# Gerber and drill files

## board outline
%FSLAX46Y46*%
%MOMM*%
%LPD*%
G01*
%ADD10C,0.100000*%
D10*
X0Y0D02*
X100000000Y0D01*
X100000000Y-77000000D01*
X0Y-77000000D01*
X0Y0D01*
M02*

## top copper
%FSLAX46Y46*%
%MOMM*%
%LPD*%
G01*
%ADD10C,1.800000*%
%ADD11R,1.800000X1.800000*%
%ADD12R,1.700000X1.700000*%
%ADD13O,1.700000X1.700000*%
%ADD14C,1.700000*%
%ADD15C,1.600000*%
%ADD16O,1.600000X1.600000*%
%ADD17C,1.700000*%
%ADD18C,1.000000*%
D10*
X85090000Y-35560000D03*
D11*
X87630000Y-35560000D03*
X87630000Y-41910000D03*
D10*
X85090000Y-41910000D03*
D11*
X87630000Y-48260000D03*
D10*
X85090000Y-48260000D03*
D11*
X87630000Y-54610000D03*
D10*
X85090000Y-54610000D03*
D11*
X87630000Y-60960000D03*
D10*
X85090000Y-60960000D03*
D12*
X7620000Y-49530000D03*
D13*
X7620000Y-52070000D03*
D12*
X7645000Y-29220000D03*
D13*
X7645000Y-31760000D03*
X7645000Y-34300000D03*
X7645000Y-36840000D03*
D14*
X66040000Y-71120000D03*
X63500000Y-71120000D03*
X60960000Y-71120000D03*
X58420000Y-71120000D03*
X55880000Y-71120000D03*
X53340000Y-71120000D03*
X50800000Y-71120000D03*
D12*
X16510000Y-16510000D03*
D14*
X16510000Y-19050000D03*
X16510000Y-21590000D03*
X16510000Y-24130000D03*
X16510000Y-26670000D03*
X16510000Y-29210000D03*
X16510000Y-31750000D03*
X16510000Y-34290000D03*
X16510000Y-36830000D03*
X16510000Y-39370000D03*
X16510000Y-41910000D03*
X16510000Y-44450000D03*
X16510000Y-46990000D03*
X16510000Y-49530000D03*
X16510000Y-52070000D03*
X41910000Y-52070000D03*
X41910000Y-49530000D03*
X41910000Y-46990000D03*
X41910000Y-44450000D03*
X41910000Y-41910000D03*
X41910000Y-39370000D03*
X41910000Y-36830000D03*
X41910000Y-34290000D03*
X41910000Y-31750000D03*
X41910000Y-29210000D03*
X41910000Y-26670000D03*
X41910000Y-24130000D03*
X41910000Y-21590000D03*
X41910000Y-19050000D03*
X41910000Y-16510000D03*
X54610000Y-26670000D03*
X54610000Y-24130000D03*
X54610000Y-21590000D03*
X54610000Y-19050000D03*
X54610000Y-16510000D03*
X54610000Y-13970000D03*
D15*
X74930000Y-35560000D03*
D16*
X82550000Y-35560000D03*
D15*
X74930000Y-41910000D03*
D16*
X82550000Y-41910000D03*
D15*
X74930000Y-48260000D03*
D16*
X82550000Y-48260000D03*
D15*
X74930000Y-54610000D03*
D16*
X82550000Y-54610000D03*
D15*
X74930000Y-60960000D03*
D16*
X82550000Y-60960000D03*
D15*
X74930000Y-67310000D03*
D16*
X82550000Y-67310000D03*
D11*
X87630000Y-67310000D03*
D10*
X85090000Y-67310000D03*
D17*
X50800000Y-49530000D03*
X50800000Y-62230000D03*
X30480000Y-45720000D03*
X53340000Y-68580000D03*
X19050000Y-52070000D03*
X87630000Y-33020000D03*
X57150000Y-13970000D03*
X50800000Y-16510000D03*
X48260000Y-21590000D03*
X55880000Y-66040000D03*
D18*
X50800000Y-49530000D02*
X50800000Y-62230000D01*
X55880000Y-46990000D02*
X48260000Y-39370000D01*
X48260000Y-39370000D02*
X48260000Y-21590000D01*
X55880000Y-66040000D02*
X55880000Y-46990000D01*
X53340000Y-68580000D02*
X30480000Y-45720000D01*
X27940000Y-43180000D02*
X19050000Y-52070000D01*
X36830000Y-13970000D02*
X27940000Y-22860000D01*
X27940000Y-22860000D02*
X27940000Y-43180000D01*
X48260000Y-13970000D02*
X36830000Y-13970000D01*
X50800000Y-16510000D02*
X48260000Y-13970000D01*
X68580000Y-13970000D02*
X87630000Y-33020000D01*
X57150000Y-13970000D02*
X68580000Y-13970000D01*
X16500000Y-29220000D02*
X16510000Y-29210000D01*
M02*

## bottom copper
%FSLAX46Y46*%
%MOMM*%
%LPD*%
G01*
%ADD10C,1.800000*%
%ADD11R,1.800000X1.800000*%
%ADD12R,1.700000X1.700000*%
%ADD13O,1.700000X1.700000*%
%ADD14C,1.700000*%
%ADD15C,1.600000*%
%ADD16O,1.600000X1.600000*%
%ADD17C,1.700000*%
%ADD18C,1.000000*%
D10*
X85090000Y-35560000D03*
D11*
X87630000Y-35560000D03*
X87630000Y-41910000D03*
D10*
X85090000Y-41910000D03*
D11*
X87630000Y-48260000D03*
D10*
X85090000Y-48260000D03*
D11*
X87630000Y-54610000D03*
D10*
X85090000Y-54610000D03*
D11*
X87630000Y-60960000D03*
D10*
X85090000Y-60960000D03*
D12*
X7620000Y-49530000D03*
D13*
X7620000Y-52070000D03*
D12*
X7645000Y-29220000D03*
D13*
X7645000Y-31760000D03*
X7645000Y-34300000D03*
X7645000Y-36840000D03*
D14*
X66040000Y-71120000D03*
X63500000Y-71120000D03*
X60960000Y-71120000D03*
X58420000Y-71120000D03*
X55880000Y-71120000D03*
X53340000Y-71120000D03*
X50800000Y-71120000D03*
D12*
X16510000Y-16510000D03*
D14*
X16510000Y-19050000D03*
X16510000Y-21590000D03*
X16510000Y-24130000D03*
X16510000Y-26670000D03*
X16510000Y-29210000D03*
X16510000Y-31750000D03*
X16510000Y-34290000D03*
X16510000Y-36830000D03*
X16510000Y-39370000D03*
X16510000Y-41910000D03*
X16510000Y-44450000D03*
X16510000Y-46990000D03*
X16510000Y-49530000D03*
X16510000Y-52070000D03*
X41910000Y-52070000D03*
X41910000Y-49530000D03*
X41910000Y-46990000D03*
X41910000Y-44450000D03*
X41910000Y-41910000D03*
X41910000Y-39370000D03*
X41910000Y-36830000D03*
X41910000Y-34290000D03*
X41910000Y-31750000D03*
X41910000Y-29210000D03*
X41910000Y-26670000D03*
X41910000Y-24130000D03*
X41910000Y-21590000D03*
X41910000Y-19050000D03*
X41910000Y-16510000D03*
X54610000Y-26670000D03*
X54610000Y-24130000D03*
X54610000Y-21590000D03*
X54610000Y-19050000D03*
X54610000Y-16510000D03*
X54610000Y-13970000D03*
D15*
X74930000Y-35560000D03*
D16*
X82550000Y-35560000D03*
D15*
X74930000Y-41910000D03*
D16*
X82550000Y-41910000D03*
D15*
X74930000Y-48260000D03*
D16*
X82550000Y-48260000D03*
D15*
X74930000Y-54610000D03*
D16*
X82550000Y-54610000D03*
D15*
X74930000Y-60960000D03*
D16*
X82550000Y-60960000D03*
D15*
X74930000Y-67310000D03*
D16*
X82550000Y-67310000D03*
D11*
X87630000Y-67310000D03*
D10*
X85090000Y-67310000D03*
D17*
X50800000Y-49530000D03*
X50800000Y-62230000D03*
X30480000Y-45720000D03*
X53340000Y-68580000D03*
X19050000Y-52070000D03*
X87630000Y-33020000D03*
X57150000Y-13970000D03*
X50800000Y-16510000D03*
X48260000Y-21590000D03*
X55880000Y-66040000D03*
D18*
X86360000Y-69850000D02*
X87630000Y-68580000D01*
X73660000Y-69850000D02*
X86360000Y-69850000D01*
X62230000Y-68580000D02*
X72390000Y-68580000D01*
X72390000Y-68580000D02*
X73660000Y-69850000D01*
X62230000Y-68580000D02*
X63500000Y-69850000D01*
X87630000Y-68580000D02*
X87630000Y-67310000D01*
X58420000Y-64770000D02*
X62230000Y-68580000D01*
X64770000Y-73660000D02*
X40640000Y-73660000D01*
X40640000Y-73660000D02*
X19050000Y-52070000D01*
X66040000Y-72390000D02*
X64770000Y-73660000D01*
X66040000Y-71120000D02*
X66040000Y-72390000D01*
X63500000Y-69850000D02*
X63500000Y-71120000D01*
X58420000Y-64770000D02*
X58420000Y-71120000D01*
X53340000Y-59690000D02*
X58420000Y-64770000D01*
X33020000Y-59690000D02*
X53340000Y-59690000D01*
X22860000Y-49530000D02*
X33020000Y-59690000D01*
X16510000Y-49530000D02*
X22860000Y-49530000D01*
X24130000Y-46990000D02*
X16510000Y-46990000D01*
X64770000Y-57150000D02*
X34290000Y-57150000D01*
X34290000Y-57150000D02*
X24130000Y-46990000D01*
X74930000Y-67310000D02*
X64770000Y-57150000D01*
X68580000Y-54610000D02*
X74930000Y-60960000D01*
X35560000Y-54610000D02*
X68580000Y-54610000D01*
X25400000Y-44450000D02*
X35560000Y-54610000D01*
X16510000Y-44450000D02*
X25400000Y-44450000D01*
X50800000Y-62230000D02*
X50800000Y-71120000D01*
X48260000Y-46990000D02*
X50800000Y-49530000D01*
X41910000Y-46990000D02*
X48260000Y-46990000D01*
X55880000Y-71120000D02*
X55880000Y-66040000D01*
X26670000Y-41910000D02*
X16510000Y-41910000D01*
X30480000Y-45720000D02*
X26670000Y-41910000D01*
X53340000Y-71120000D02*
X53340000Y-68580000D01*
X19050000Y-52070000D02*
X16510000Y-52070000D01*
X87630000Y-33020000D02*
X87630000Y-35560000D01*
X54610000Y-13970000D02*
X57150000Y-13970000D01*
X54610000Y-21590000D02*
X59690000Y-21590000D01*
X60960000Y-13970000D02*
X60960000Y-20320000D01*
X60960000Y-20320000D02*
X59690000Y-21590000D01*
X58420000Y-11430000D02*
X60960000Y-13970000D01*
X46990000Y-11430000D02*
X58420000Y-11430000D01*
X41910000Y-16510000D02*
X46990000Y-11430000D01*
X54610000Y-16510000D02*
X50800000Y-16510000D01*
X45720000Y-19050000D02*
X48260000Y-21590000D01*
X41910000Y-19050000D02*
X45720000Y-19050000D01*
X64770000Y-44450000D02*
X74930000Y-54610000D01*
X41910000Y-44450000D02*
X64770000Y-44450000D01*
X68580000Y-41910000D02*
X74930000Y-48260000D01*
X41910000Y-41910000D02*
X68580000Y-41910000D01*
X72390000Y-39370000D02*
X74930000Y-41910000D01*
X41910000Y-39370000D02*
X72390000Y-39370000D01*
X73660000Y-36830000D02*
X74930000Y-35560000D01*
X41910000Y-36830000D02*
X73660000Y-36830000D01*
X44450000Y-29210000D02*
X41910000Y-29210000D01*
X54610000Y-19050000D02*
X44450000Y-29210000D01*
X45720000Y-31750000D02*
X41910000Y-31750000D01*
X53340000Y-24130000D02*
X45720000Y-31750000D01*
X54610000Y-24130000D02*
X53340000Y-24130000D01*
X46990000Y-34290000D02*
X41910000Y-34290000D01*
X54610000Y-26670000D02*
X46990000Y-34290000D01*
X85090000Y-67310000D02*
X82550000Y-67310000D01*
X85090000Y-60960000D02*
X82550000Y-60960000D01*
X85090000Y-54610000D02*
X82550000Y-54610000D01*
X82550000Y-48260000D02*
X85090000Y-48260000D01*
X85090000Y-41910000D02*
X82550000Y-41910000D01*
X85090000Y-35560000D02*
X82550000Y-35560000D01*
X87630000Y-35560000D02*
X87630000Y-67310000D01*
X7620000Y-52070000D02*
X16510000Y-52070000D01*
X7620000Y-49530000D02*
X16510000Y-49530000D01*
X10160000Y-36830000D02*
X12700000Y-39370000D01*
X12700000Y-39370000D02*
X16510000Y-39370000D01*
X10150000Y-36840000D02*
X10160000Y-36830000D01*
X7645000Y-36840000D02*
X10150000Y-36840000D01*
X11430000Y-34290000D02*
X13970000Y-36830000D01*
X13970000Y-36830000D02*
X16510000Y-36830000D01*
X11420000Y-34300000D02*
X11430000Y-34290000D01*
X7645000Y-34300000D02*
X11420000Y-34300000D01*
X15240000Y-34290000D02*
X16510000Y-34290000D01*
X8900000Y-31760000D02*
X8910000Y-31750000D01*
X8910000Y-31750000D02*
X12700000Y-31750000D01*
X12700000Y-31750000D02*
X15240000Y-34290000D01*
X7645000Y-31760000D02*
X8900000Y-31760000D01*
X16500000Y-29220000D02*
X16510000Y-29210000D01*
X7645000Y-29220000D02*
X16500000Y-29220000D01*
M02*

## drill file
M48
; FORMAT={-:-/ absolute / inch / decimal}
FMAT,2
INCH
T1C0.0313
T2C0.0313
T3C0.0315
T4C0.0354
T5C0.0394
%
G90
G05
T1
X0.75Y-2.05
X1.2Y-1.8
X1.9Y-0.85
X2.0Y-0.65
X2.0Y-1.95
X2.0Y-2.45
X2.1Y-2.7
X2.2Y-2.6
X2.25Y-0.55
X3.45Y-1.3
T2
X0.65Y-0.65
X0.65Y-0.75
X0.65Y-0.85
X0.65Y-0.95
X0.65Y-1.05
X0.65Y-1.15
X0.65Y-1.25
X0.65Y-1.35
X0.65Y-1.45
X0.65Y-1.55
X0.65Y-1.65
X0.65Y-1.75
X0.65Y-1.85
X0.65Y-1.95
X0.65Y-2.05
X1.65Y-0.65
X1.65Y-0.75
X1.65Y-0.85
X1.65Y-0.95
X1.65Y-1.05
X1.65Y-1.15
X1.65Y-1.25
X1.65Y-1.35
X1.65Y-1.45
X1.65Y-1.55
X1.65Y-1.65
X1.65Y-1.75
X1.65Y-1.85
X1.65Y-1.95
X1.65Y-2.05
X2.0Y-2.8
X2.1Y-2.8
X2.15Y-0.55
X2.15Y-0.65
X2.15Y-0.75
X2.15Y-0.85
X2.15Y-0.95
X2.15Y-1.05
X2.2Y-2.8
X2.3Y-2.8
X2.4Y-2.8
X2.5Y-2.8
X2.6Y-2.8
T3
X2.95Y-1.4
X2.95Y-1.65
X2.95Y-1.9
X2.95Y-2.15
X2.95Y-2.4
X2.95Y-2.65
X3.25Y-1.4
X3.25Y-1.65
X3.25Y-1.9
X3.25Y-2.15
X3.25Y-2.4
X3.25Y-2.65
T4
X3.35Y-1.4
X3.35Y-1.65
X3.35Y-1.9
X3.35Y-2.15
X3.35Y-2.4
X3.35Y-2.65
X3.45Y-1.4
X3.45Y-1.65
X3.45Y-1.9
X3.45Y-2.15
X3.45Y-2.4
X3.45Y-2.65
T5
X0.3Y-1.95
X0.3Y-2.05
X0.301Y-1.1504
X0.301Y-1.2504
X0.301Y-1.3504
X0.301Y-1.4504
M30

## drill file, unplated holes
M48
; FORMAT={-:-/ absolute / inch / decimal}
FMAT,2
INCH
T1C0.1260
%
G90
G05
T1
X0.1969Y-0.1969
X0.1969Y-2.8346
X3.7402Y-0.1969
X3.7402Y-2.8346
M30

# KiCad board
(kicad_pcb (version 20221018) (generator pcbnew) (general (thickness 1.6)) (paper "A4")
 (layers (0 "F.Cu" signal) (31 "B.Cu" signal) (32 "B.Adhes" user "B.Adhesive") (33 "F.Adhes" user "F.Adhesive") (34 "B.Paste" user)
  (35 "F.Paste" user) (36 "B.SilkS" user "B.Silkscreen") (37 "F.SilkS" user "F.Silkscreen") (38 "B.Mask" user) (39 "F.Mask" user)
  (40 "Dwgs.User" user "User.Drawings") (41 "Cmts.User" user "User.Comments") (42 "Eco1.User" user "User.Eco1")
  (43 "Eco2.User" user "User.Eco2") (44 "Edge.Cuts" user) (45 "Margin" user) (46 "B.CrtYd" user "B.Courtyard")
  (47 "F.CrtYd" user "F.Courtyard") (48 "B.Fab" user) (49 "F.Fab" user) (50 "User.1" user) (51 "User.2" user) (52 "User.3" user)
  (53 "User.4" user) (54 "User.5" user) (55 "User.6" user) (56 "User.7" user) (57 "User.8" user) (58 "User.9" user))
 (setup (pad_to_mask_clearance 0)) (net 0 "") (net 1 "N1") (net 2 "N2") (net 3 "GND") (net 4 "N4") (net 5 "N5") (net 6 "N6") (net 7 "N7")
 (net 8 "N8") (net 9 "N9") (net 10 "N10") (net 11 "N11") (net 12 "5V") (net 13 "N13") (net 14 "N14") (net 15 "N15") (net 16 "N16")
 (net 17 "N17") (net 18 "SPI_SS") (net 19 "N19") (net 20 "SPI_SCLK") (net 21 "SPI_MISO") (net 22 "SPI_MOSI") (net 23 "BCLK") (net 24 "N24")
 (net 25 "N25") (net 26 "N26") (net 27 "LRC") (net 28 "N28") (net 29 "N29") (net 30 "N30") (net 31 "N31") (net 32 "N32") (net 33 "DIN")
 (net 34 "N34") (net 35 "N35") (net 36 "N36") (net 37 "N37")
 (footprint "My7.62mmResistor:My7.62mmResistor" (layer "F.Cu") (at 74.93 60.96)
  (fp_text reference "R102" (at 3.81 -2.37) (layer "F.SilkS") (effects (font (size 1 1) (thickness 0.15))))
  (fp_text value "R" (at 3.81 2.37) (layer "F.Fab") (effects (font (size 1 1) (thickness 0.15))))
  (pad "1" thru_hole circle (at 0 0) (size 1.6 1.6) (drill 0.8) (layers "*.Cu" "*.Mask") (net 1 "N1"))
  (pad "2" thru_hole oval (at 7.62 0) (size 1.6 1.6) (drill 0.8) (layers "*.Cu" "*.Mask") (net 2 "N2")))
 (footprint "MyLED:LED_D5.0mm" (layer "F.Cu") (at 86.36 54.61 180)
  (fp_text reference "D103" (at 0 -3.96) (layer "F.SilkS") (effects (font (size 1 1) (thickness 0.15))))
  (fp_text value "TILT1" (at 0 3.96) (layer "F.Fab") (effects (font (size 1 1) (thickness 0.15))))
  (pad "1" thru_hole rect (at -1.27 0 180) (size 1.8 1.8) (drill 0.9) (layers "*.Cu" "*.Mask") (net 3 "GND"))
  (pad "2" thru_hole circle (at 1.27 0 180) (size 1.8 1.8) (drill 0.9) (layers "*.Cu" "*.Mask") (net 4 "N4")))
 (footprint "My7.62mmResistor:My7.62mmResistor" (layer "F.Cu") (at 74.93 48.26)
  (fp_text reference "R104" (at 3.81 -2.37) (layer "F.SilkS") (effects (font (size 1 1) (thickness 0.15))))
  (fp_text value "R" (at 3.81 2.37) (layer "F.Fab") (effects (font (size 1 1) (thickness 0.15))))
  (pad "1" thru_hole circle (at 0 0) (size 1.6 1.6) (drill 0.8) (layers "*.Cu" "*.Mask") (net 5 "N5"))
  (pad "2" thru_hole oval (at 7.62 0) (size 1.6 1.6) (drill 0.8) (layers "*.Cu" "*.Mask") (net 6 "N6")))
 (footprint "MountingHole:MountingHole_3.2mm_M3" (layer "F.Cu") (at 95 5)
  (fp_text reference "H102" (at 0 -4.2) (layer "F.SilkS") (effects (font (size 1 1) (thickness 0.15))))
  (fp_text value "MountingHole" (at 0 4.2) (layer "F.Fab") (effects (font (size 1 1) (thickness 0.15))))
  (pad "" np_thru_hole circle (at 0 0) (size 3.2 3.2) (drill 3.2) (layers "*.Cu" "*.Mask")))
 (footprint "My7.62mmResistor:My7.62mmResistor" (layer "F.Cu") (at 74.93 54.61)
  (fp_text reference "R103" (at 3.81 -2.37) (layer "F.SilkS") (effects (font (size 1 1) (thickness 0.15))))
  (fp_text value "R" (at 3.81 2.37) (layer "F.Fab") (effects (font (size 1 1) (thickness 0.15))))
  (pad "1" thru_hole circle (at 0 0) (size 1.6 1.6) (drill 0.8) (layers "*.Cu" "*.Mask") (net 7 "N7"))
  (pad "2" thru_hole oval (at 7.62 0) (size 1.6 1.6) (drill 0.8) (layers "*.Cu" "*.Mask") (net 4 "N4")))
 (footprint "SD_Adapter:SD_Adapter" (layer "F.Cu") (at 64.77 19.05 -90)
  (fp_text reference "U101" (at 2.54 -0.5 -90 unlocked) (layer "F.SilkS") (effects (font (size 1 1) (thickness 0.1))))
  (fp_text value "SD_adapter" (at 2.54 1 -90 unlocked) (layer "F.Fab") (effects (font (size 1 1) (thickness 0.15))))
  (pad "1" thru_hole circle (at 7.62 10.16 270) (size 1.7 1.7) (drill 0.794) (layers "*.Cu" "*.Mask") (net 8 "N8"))
  (pad "2" thru_hole circle (at 5.08 10.16 270) (size 1.7 1.7) (drill 0.794) (layers "*.Cu" "*.Mask") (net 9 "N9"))
  (pad "3" thru_hole circle (at 2.54 10.16 270) (size 1.7 1.7) (drill 0.794) (layers "*.Cu" "*.Mask") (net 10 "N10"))
  (pad "4" thru_hole circle (at 0 10.16 270) (size 1.7 1.7) (drill 0.794) (layers "*.Cu" "*.Mask") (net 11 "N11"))
  (pad "5" thru_hole circle (at -2.54 10.16 270) (size 1.7 1.7) (drill 0.794) (layers "*.Cu" "*.Mask") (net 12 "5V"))
  (pad "6" thru_hole circle (at -5.08 10.16 270) (size 1.7 1.7) (drill 0.794) (layers "*.Cu" "*.Mask") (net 3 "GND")))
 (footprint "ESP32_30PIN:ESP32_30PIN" (layer "F.Cu") (at 29.21 34.29)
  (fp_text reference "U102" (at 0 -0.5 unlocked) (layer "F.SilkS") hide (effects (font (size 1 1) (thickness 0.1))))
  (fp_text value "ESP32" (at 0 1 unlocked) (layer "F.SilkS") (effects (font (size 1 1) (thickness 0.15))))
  (pad "1" thru_hole rect (at -12.7 -17.78) (size 1.7 1.7) (drill 0.794) (layers "*.Cu" "*.Mask") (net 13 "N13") (solder_mask_margin 0.102))
  (pad "2" thru_hole circle (at -12.7 -15.24) (size 1.7 1.7) (drill 0.794) (layers "*.Cu" "*.Mask") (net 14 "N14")
   (solder_mask_margin 0.102))
  (pad "3" thru_hole circle (at -12.7 -12.7) (size 1.7 1.7) (drill 0.794) (layers "*.Cu" "*.Mask") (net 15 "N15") (solder_mask_margin 0.102))
  (pad "4" thru_hole circle (at -12.7 -10.16) (size 1.7 1.7) (drill 0.794) (layers "*.Cu" "*.Mask") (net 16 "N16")
   (solder_mask_margin 0.102))
  (pad "5" thru_hole circle (at -12.7 -7.62) (size 1.7 1.7) (drill 0.794) (layers "*.Cu" "*.Mask") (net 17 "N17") (solder_mask_margin 0.102))
  (pad "6" thru_hole circle (at -12.7 -5.08) (size 1.7 1.7) (drill 0.794) (layers "*.Cu" "*.Mask") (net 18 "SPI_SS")
   (solder_mask_margin 0.102))
  (pad "7" thru_hole circle (at -12.7 -2.54) (size 1.7 1.7) (drill 0.794) (layers "*.Cu" "*.Mask") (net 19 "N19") (solder_mask_margin 0.102))
  (pad "8" thru_hole circle (at -12.7 0) (size 1.7 1.7) (drill 0.794) (layers "*.Cu" "*.Mask") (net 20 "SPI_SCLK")
   (solder_mask_margin 0.102))
  (pad "9" thru_hole circle (at -12.7 2.54) (size 1.7 1.7) (drill 0.794) (layers "*.Cu" "*.Mask") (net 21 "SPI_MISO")
   (solder_mask_margin 0.102))
  (pad "10" thru_hole circle (at -12.7 5.08) (size 1.7 1.7) (drill 0.794) (layers "*.Cu" "*.Mask") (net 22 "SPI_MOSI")
   (solder_mask_margin 0.102))
  (pad "11" thru_hole circle (at -12.7 7.62) (size 1.7 1.7) (drill 0.794) (layers "*.Cu" "*.Mask") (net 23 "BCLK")
   (solder_mask_margin 0.102))
  (pad "12" thru_hole circle (at -12.7 10.16) (size 1.7 1.7) (drill 0.794) (layers "*.Cu" "*.Mask") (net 1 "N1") (solder_mask_margin 0.102))
  (pad "13" thru_hole circle (at -12.7 12.7) (size 1.7 1.7) (drill 0.794) (layers "*.Cu" "*.Mask") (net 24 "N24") (solder_mask_margin 0.102))
  (pad "14" thru_hole circle (at -12.7 15.24) (size 1.7 1.7) (drill 0.794) (layers "*.Cu" "*.Mask") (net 3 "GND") (solder_mask_margin 0.102))
  (pad "15" thru_hole circle (at -12.7 17.78) (size 1.7 1.7) (drill 0.794) (layers "*.Cu" "*.Mask") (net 12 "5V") (solder_mask_margin 0.102))
  (pad "16" thru_hole circle (at 12.7 17.78) (size 1.7 1.7) (drill 0.794) (layers "*.Cu" "*.Mask") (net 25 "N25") (solder_mask_margin 0.102))
  (pad "17" thru_hole circle (at 12.7 15.24) (size 1.7 1.7) (drill 0.794) (layers "*.Cu" "*.Mask") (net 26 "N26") (solder_mask_margin 0.102))
  (pad "18" thru_hole circle (at 12.7 12.7) (size 1.7 1.7) (drill 0.794) (layers "*.Cu" "*.Mask") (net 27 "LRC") (solder_mask_margin 0.102))
  (pad "19" thru_hole circle (at 12.7 10.16) (size 1.7 1.7) (drill 0.794) (layers "*.Cu" "*.Mask") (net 7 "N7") (solder_mask_margin 0.102))
  (pad "20" thru_hole circle (at 12.7 7.62) (size 1.7 1.7) (drill 0.794) (layers "*.Cu" "*.Mask") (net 5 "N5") (solder_mask_margin 0.102))
  (pad "21" thru_hole circle (at 12.7 5.08) (size 1.7 1.7) (drill 0.794) (layers "*.Cu" "*.Mask") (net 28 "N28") (solder_mask_margin 0.102))
  (pad "22" thru_hole circle (at 12.7 2.54) (size 1.7 1.7) (drill 0.794) (layers "*.Cu" "*.Mask") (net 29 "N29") (solder_mask_margin 0.102))
  (pad "23" thru_hole circle (at 12.7 0) (size 1.7 1.7) (drill 0.794) (layers "*.Cu" "*.Mask") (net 8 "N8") (solder_mask_margin 0.102))
  (pad "24" thru_hole circle (at 12.7 -2.54) (size 1.7 1.7) (drill 0.794) (layers "*.Cu" "*.Mask") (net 9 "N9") (solder_mask_margin 0.102))
  (pad "25" thru_hole circle (at 12.7 -5.08) (size 1.7 1.7) (drill 0.794) (layers "*.Cu" "*.Mask") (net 11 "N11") (solder_mask_margin 0.102))
  (pad "26" thru_hole circle (at 12.7 -7.62) (size 1.7 1.7) (drill 0.794) (layers "*.Cu" "*.Mask") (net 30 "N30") (solder_mask_margin 0.102))
  (pad "27" thru_hole circle (at 12.7 -10.16) (size 1.7 1.7) (drill 0.794) (layers "*.Cu" "*.Mask") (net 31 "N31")
   (solder_mask_margin 0.102))
  (pad "28" thru_hole circle (at 12.7 -12.7) (size 1.7 1.7) (drill 0.794) (layers "*.Cu" "*.Mask") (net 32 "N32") (solder_mask_margin 0.102))
  (pad "29" thru_hole circle (at 12.7 -15.24) (size 1.7 1.7) (drill 0.794) (layers "*.Cu" "*.Mask") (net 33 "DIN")
   (solder_mask_margin 0.102))
  (pad "30" thru_hole circle (at 12.7 -17.78) (size 1.7 1.7) (drill 0.794) (layers "*.Cu" "*.Mask") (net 10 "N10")
   (solder_mask_margin 0.102)))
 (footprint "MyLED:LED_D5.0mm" (layer "F.Cu") (at 86.36 60.96 180)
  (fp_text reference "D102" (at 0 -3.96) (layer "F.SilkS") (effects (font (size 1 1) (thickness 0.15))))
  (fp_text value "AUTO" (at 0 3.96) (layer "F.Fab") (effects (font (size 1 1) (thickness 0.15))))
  (pad "1" thru_hole rect (at -1.27 0 180) (size 1.8 1.8) (drill 0.9) (layers "*.Cu" "*.Mask") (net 3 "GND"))
  (pad "2" thru_hole circle (at 1.27 0 180) (size 1.8 1.8) (drill 0.9) (layers "*.Cu" "*.Mask") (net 2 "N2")))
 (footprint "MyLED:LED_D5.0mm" (layer "F.Cu") (at 86.36 41.91 180)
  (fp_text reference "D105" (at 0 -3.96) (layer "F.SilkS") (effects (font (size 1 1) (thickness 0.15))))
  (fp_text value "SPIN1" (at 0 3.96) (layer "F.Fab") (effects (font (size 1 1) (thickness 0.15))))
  (pad "1" thru_hole rect (at -1.27 0 180) (size 1.8 1.8) (drill 0.9) (layers "*.Cu" "*.Mask") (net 3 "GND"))
  (pad "2" thru_hole circle (at 1.27 0 180) (size 1.8 1.8) (drill 0.9) (layers "*.Cu" "*.Mask") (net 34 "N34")))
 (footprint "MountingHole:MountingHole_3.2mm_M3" (layer "F.Cu") (at 95 72)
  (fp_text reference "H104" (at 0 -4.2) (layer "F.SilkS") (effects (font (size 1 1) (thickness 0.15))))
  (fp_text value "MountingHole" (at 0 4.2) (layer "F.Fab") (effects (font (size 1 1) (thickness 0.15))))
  (pad "" np_thru_hole circle (at 0 0) (size 3.2 3.2) (drill 3.2) (layers "*.Cu" "*.Mask")))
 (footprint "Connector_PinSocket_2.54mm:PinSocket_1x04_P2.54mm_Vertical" (layer "F.Cu") (at 7.645 29.22)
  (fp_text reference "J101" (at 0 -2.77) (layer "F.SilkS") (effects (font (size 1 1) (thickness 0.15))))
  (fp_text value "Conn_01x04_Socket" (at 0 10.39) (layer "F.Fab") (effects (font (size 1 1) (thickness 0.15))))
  (pad "1" thru_hole rect (at 0 0) (size 1.7 1.7) (drill 1) (layers "*.Cu" "*.Mask") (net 18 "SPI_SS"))
  (pad "2" thru_hole oval (at 0 2.54) (size 1.7 1.7) (drill 1) (layers "*.Cu" "*.Mask") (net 20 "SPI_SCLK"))
  (pad "3" thru_hole oval (at 0 5.08) (size 1.7 1.7) (drill 1) (layers "*.Cu" "*.Mask") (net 21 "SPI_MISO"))
  (pad "4" thru_hole oval (at 0 7.62) (size 1.7 1.7) (drill 1) (layers "*.Cu" "*.Mask") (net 22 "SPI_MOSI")))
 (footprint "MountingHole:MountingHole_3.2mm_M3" (layer "F.Cu") (at 5 72)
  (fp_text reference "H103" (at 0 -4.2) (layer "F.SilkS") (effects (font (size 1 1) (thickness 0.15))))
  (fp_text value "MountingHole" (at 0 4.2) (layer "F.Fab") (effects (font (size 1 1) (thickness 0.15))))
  (pad "" np_thru_hole circle (at 0 0) (size 3.2 3.2) (drill 3.2) (layers "*.Cu" "*.Mask")))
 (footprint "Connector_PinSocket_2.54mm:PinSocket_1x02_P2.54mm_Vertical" (layer "F.Cu") (at 7.62 49.53)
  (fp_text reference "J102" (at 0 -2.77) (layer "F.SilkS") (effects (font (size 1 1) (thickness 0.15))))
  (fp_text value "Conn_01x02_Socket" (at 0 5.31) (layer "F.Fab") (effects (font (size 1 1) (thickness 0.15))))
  (pad "1" thru_hole rect (at 0 0) (size 1.7 1.7) (drill 1) (layers "*.Cu" "*.Mask") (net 3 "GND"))
  (pad "2" thru_hole oval (at 0 2.54) (size 1.7 1.7) (drill 1) (layers "*.Cu" "*.Mask") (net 12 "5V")))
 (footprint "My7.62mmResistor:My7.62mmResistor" (layer "F.Cu") (at 74.93 35.56)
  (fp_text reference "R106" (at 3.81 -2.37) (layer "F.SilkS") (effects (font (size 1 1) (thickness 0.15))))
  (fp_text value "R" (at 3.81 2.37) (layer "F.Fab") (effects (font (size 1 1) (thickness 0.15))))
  (pad "1" thru_hole circle (at 0 0) (size 1.6 1.6) (drill 0.8) (layers "*.Cu" "*.Mask") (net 29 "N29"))
  (pad "2" thru_hole oval (at 7.62 0) (size 1.6 1.6) (drill 0.8) (layers "*.Cu" "*.Mask") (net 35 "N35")))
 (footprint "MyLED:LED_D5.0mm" (layer "F.Cu") (at 86.36 67.31 180)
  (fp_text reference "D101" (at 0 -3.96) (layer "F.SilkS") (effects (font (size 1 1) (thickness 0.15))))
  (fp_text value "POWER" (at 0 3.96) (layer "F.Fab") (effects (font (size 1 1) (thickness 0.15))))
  (pad "1" thru_hole rect (at -1.27 0 180) (size 1.8 1.8) (drill 0.9) (layers "*.Cu" "*.Mask") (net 3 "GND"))
  (pad "2" thru_hole circle (at 1.27 0 180) (size 1.8 1.8) (drill 0.9) (layers "*.Cu" "*.Mask") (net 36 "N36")))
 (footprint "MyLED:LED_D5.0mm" (layer "F.Cu") (at 86.36 35.56 180)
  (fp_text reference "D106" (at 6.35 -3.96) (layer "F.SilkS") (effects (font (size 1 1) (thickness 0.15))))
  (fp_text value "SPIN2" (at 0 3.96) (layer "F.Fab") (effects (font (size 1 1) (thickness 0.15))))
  (pad "1" thru_hole rect (at -1.27 0 180) (size 1.8 1.8) (drill 0.9) (layers "*.Cu" "*.Mask") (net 3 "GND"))
  (pad "2" thru_hole circle (at 1.27 0 180) (size 1.8 1.8) (drill 0.9) (layers "*.Cu" "*.Mask") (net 35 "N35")))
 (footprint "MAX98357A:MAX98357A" (layer "F.Cu") (at 58.42 77.47 180)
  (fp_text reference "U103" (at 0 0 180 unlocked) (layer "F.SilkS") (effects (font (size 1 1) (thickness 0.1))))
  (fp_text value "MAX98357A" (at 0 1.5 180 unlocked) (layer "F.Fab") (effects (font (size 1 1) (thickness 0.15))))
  (pad "1" thru_hole circle (at -7.62 6.35 180) (size 1.7 1.7) (drill 0.794) (layers "*.Cu" "*.Mask") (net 12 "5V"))
  (pad "2" thru_hole circle (at -5.08 6.35 180) (size 1.7 1.7) (drill 0.794) (layers "*.Cu" "*.Mask") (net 3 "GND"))
  (pad "3" thru_hole circle (at -2.54 6.35 180) (size 1.7 1.7) (drill 0.794) (layers "*.Cu" "*.Mask") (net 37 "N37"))
  (pad "4" thru_hole circle (at 0 6.35 180) (size 1.7 1.7) (drill 0.794) (layers "*.Cu" "*.Mask") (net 3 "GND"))
  (pad "5" thru_hole circle (at 2.54 6.35 180) (size 1.7 1.7) (drill 0.794) (layers "*.Cu" "*.Mask") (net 33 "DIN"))
  (pad "6" thru_hole circle (at 5.08 6.35 180) (size 1.7 1.7) (drill 0.794) (layers "*.Cu" "*.Mask") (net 23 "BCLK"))
  (pad "7" thru_hole circle (at 7.62 6.35 180) (size 1.7 1.7) (drill 0.794) (layers "*.Cu" "*.Mask") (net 27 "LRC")))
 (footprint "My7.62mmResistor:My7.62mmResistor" (layer "F.Cu") (at 74.93 41.91)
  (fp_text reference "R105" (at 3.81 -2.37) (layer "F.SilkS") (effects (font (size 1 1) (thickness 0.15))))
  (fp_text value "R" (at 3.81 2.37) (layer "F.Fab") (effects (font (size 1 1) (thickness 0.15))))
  (pad "1" thru_hole circle (at 0 0) (size 1.6 1.6) (drill 0.8) (layers "*.Cu" "*.Mask") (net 28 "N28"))
  (pad "2" thru_hole oval (at 7.62 0) (size 1.6 1.6) (drill 0.8) (layers "*.Cu" "*.Mask") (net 34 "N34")))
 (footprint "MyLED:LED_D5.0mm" (layer "F.Cu") (at 86.36 48.26 180)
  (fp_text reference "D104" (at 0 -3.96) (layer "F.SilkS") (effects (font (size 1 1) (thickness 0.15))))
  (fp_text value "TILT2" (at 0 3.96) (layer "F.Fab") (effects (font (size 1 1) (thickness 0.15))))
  (pad "1" thru_hole rect (at -1.27 0 180) (size 1.8 1.8) (drill 0.9) (layers "*.Cu" "*.Mask") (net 3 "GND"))
  (pad "2" thru_hole circle (at 1.27 0 180) (size 1.8 1.8) (drill 0.9) (layers "*.Cu" "*.Mask") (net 6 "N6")))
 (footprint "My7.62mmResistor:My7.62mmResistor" (layer "F.Cu") (at 74.93 67.31)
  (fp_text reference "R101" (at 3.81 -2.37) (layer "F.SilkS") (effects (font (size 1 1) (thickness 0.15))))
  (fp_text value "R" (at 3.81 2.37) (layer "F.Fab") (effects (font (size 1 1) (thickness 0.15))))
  (pad "1" thru_hole circle (at 0 0) (size 1.6 1.6) (drill 0.8) (layers "*.Cu" "*.Mask") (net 24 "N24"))
  (pad "2" thru_hole oval (at 7.62 0) (size 1.6 1.6) (drill 0.8) (layers "*.Cu" "*.Mask") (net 36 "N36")))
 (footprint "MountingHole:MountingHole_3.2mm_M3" (layer "F.Cu") (at 5 5)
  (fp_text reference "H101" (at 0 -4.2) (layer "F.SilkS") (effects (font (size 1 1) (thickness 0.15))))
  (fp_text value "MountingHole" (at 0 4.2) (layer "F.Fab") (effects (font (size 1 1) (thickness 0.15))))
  (pad "" np_thru_hole circle (at 0 0) (size 3.2 3.2) (drill 3.2) (layers "*.Cu" "*.Mask")))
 (gr_rect (start 0 0) (end 100 77) (stroke (width 0.1) (type default)) (fill none) (layer "Edge.Cuts"))
 (segment (start 57.15 13.97) (end 68.58 13.97) (width 1) (layer "F.Cu") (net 3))
 (segment (start 68.58 13.97) (end 87.63 33.02) (width 1) (layer "F.Cu") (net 3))
 (via (at 57.15 13.97) (size 1.7) (drill 0.794) (layers "F.Cu" "B.Cu") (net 3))
 (via (at 87.63 33.02) (size 1.7) (drill 0.794) (layers "F.Cu" "B.Cu") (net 3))
 (segment (start 87.63 68.58) (end 87.63 67.31) (width 1) (layer "B.Cu") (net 3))
 (segment (start 63.5 69.85) (end 63.5 71.12) (width 1) (layer "B.Cu") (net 3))
 (segment (start 73.66 69.85) (end 86.36 69.85) (width 1) (layer "B.Cu") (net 3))
 (segment (start 87.63 35.56) (end 87.63 67.31) (width 1) (layer "B.Cu") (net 3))
 (segment (start 7.62 49.53) (end 16.51 49.53) (width 1) (layer "B.Cu") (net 3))
 (segment (start 58.42 64.77) (end 62.23 68.58) (width 1) (layer "B.Cu") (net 3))
 (segment (start 86.36 69.85) (end 87.63 68.58) (width 1) (layer "B.Cu") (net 3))
 (segment (start 33.02 59.69) (end 53.34 59.69) (width 1) (layer "B.Cu") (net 3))
 (segment (start 53.34 59.69) (end 58.42 64.77) (width 1) (layer "B.Cu") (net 3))
 (segment (start 72.39 68.58) (end 73.66 69.85) (width 1) (layer "B.Cu") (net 3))
 (segment (start 87.63 33.02) (end 87.63 35.56) (width 1) (layer "B.Cu") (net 3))
 (segment (start 22.86 49.53) (end 33.02 59.69) (width 1) (layer "B.Cu") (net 3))
 (segment (start 62.23 68.58) (end 63.5 69.85) (width 1) (layer "B.Cu") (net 3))
 (segment (start 62.23 68.58) (end 72.39 68.58) (width 1) (layer "B.Cu") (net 3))
 (segment (start 54.61 13.97) (end 57.15 13.97) (width 1) (layer "B.Cu") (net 3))
 (segment (start 58.42 64.77) (end 58.42 71.12) (width 1) (layer "B.Cu") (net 3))
 (segment (start 16.51 49.53) (end 22.86 49.53) (width 1) (layer "B.Cu") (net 3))
 (segment (start 85.09 67.31) (end 82.55 67.31) (width 1) (layer "B.Cu") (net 36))
 (segment (start 50.8 16.51) (end 48.26 13.97) (width 1) (layer "F.Cu") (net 12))
 (segment (start 48.26 13.97) (end 36.83 13.97) (width 1) (layer "F.Cu") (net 12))
 (segment (start 27.94 43.18) (end 19.05 52.07) (width 1) (layer "F.Cu") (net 12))
 (segment (start 36.83 13.97) (end 27.94 22.86) (width 1) (layer "F.Cu") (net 12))
 (segment (start 27.94 22.86) (end 27.94 43.18) (width 1) (layer "F.Cu") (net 12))
 (via (at 19.05 52.07) (size 1.7) (drill 0.794) (layers "F.Cu" "B.Cu") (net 12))
 (via (at 50.8 16.51) (size 1.7) (drill 0.794) (layers "F.Cu" "B.Cu") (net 12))
 (segment (start 7.62 52.07) (end 16.51 52.07) (width 1) (layer "B.Cu") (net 12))
 (segment (start 40.64 73.66) (end 19.05 52.07) (width 1) (layer "B.Cu") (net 12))
 (segment (start 19.05 52.07) (end 16.51 52.07) (width 1) (layer "B.Cu") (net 12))
 (segment (start 66.04 72.39) (end 64.77 73.66) (width 1) (layer "B.Cu") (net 12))
 (segment (start 64.77 73.66) (end 40.64 73.66) (width 1) (layer "B.Cu") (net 12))
 (segment (start 54.61 16.51) (end 50.8 16.51) (width 1) (layer "B.Cu") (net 12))
 (segment (start 66.04 71.12) (end 66.04 72.39) (width 1) (layer "B.Cu") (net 12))
 (segment (start 41.91 44.45) (end 64.77 44.45) (width 1) (layer "B.Cu") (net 7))
 (segment (start 64.77 44.45) (end 74.93 54.61) (width 1) (layer "B.Cu") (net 7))
 (segment (start 68.58 41.91) (end 74.93 48.26) (width 1) (layer "B.Cu") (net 5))
 (segment (start 41.91 41.91) (end 68.58 41.91) (width 1) (layer "B.Cu") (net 5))
 (segment (start 85.09 60.96) (end 82.55 60.96) (width 1) (layer "B.Cu") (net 2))
 (segment (start 41.91 39.37) (end 72.39 39.37) (width 1) (layer "B.Cu") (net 28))
 (segment (start 72.39 39.37) (end 74.93 41.91) (width 1) (layer "B.Cu") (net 28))
 (segment (start 85.09 54.61) (end 82.55 54.61) (width 1) (layer "B.Cu") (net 4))
 (segment (start 73.66 36.83) (end 74.93 35.56) (width 1) (layer "B.Cu") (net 29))
 (segment (start 41.91 36.83) (end 73.66 36.83) (width 1) (layer "B.Cu") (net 29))
 (segment (start 82.55 48.26) (end 85.09 48.26) (width 1) (layer "B.Cu") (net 6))
 (segment (start 85.09 41.91) (end 82.55 41.91) (width 1) (layer "B.Cu") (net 34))
 (segment (start 85.09 35.56) (end 82.55 35.56) (width 1) (layer "B.Cu") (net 35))
 (segment (start 46.99 34.29) (end 41.91 34.29) (width 1) (layer "B.Cu") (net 8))
 (segment (start 54.61 26.67) (end 46.99 34.29) (width 1) (layer "B.Cu") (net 8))
 (segment (start 53.34 24.13) (end 45.72 31.75) (width 1) (layer "B.Cu") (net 9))
 (segment (start 54.61 24.13) (end 53.34 24.13) (width 1) (layer "B.Cu") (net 9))
 (segment (start 45.72 31.75) (end 41.91 31.75) (width 1) (layer "B.Cu") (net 9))
 (segment (start 46.99 11.43) (end 58.42 11.43) (width 1) (layer "B.Cu") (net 10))
 (segment (start 41.91 16.51) (end 46.99 11.43) (width 1) (layer "B.Cu") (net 10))
 (segment (start 60.96 13.97) (end 60.96 20.32) (width 1) (layer "B.Cu") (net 10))
 (segment (start 58.42 11.43) (end 60.96 13.97) (width 1) (layer "B.Cu") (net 10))
 (segment (start 60.96 20.32) (end 59.69 21.59) (width 1) (layer "B.Cu") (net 10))
 (segment (start 54.61 21.59) (end 59.69 21.59) (width 1) (layer "B.Cu") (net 10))
 (segment (start 44.45 29.21) (end 41.91 29.21) (width 1) (layer "B.Cu") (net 11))
 (segment (start 54.61 19.05) (end 44.45 29.21) (width 1) (layer "B.Cu") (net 11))
 (segment (start 16.5 29.22) (end 16.51 29.21) (width 1) (layer "F.Cu") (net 18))
 (segment (start 7.645 29.22) (end 16.5 29.22) (width 1) (layer "B.Cu") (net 18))
 (segment (start 16.5 29.22) (end 16.51 29.21) (width 1) (layer "B.Cu") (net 18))
 (segment (start 8.9 31.76) (end 8.91 31.75) (width 1) (layer "B.Cu") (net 20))
 (segment (start 7.645 31.76) (end 8.9 31.76) (width 1) (layer "B.Cu") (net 20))
 (segment (start 8.91 31.75) (end 12.7 31.75) (width 1) (layer "B.Cu") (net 20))
 (segment (start 12.7 31.75) (end 15.24 34.29) (width 1) (layer "B.Cu") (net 20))
 (segment (start 15.24 34.29) (end 16.51 34.29) (width 1) (layer "B.Cu") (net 20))
 (segment (start 7.645 34.3) (end 11.42 34.3) (width 1) (layer "B.Cu") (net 21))
 (segment (start 11.43 34.29) (end 13.97 36.83) (width 1) (layer "B.Cu") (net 21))
 (segment (start 11.42 34.3) (end 11.43 34.29) (width 1) (layer "B.Cu") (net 21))
 (segment (start 13.97 36.83) (end 16.51 36.83) (width 1) (layer "B.Cu") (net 21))
 (segment (start 10.16 36.83) (end 12.7 39.37) (width 1) (layer "B.Cu") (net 22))
 (segment (start 10.15 36.84) (end 10.16 36.83) (width 1) (layer "B.Cu") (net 22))
 (segment (start 7.645 36.84) (end 10.15 36.84) (width 1) (layer "B.Cu") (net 22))
 (segment (start 12.7 39.37) (end 16.51 39.37) (width 1) (layer "B.Cu") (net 22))
 (segment (start 53.34 68.58) (end 30.48 45.72) (width 1) (layer "F.Cu") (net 23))
 (via (at 53.34 68.58) (size 1.7) (drill 0.794) (layers "F.Cu" "B.Cu") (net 23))
 (via (at 30.48 45.72) (size 1.7) (drill 0.794) (layers "F.Cu" "B.Cu") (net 23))
 (segment (start 30.48 45.72) (end 26.67 41.91) (width 1) (layer "B.Cu") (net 23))
 (segment (start 53.34 71.12) (end 53.34 68.58) (width 1) (layer "B.Cu") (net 23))
 (segment (start 26.67 41.91) (end 16.51 41.91) (width 1) (layer "B.Cu") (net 23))
 (segment (start 50.8 49.53) (end 50.8 62.23) (width 1) (layer "F.Cu") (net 27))
 (via (at 50.8 49.53) (size 1.7) (drill 0.794) (layers "F.Cu" "B.Cu") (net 27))
 (via (at 50.8 62.23) (size 1.7) (drill 0.794) (layers "F.Cu" "B.Cu") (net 27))
 (segment (start 41.91 46.99) (end 48.26 46.99) (width 1) (layer "B.Cu") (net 27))
 (segment (start 50.8 62.23) (end 50.8 71.12) (width 1) (layer "B.Cu") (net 27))
 (segment (start 48.26 46.99) (end 50.8 49.53) (width 1) (layer "B.Cu") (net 27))
 (segment (start 55.88 66.04) (end 55.88 46.99) (width 1) (layer "F.Cu") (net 33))
 (segment (start 48.26 39.37) (end 48.26 21.59) (width 1) (layer "F.Cu") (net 33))
 (segment (start 55.88 46.99) (end 48.26 39.37) (width 1) (layer "F.Cu") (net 33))
 (via (at 48.26 21.59) (size 1.7) (drill 0.794) (layers "F.Cu" "B.Cu") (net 33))
 (via (at 55.88 66.04) (size 1.7) (drill 0.794) (layers "F.Cu" "B.Cu") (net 33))
 (segment (start 45.72 19.05) (end 48.26 21.59) (width 1) (layer "B.Cu") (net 33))
 (segment (start 41.91 19.05) (end 45.72 19.05) (width 1) (layer "B.Cu") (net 33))
 (segment (start 55.88 71.12) (end 55.88 66.04) (width 1) (layer "B.Cu") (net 33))
 (segment (start 24.13 46.99) (end 16.51 46.99) (width 1) (layer "B.Cu") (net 24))
 (segment (start 74.93 67.31) (end 64.77 57.15) (width 1) (layer "B.Cu") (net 24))
 (segment (start 64.77 57.15) (end 34.29 57.15) (width 1) (layer "B.Cu") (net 24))
 (segment (start 34.29 57.15) (end 24.13 46.99) (width 1) (layer "B.Cu") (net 24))
 (segment (start 25.4 44.45) (end 35.56 54.61) (width 1) (layer "B.Cu") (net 1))
 (segment (start 16.51 44.45) (end 25.4 44.45) (width 1) (layer "B.Cu") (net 1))
 (segment (start 35.56 54.61) (end 68.58 54.61) (width 1) (layer "B.Cu") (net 1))
 (segment (start 68.58 54.61) (end 74.93 60.96) (width 1) (layer "B.Cu") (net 1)))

